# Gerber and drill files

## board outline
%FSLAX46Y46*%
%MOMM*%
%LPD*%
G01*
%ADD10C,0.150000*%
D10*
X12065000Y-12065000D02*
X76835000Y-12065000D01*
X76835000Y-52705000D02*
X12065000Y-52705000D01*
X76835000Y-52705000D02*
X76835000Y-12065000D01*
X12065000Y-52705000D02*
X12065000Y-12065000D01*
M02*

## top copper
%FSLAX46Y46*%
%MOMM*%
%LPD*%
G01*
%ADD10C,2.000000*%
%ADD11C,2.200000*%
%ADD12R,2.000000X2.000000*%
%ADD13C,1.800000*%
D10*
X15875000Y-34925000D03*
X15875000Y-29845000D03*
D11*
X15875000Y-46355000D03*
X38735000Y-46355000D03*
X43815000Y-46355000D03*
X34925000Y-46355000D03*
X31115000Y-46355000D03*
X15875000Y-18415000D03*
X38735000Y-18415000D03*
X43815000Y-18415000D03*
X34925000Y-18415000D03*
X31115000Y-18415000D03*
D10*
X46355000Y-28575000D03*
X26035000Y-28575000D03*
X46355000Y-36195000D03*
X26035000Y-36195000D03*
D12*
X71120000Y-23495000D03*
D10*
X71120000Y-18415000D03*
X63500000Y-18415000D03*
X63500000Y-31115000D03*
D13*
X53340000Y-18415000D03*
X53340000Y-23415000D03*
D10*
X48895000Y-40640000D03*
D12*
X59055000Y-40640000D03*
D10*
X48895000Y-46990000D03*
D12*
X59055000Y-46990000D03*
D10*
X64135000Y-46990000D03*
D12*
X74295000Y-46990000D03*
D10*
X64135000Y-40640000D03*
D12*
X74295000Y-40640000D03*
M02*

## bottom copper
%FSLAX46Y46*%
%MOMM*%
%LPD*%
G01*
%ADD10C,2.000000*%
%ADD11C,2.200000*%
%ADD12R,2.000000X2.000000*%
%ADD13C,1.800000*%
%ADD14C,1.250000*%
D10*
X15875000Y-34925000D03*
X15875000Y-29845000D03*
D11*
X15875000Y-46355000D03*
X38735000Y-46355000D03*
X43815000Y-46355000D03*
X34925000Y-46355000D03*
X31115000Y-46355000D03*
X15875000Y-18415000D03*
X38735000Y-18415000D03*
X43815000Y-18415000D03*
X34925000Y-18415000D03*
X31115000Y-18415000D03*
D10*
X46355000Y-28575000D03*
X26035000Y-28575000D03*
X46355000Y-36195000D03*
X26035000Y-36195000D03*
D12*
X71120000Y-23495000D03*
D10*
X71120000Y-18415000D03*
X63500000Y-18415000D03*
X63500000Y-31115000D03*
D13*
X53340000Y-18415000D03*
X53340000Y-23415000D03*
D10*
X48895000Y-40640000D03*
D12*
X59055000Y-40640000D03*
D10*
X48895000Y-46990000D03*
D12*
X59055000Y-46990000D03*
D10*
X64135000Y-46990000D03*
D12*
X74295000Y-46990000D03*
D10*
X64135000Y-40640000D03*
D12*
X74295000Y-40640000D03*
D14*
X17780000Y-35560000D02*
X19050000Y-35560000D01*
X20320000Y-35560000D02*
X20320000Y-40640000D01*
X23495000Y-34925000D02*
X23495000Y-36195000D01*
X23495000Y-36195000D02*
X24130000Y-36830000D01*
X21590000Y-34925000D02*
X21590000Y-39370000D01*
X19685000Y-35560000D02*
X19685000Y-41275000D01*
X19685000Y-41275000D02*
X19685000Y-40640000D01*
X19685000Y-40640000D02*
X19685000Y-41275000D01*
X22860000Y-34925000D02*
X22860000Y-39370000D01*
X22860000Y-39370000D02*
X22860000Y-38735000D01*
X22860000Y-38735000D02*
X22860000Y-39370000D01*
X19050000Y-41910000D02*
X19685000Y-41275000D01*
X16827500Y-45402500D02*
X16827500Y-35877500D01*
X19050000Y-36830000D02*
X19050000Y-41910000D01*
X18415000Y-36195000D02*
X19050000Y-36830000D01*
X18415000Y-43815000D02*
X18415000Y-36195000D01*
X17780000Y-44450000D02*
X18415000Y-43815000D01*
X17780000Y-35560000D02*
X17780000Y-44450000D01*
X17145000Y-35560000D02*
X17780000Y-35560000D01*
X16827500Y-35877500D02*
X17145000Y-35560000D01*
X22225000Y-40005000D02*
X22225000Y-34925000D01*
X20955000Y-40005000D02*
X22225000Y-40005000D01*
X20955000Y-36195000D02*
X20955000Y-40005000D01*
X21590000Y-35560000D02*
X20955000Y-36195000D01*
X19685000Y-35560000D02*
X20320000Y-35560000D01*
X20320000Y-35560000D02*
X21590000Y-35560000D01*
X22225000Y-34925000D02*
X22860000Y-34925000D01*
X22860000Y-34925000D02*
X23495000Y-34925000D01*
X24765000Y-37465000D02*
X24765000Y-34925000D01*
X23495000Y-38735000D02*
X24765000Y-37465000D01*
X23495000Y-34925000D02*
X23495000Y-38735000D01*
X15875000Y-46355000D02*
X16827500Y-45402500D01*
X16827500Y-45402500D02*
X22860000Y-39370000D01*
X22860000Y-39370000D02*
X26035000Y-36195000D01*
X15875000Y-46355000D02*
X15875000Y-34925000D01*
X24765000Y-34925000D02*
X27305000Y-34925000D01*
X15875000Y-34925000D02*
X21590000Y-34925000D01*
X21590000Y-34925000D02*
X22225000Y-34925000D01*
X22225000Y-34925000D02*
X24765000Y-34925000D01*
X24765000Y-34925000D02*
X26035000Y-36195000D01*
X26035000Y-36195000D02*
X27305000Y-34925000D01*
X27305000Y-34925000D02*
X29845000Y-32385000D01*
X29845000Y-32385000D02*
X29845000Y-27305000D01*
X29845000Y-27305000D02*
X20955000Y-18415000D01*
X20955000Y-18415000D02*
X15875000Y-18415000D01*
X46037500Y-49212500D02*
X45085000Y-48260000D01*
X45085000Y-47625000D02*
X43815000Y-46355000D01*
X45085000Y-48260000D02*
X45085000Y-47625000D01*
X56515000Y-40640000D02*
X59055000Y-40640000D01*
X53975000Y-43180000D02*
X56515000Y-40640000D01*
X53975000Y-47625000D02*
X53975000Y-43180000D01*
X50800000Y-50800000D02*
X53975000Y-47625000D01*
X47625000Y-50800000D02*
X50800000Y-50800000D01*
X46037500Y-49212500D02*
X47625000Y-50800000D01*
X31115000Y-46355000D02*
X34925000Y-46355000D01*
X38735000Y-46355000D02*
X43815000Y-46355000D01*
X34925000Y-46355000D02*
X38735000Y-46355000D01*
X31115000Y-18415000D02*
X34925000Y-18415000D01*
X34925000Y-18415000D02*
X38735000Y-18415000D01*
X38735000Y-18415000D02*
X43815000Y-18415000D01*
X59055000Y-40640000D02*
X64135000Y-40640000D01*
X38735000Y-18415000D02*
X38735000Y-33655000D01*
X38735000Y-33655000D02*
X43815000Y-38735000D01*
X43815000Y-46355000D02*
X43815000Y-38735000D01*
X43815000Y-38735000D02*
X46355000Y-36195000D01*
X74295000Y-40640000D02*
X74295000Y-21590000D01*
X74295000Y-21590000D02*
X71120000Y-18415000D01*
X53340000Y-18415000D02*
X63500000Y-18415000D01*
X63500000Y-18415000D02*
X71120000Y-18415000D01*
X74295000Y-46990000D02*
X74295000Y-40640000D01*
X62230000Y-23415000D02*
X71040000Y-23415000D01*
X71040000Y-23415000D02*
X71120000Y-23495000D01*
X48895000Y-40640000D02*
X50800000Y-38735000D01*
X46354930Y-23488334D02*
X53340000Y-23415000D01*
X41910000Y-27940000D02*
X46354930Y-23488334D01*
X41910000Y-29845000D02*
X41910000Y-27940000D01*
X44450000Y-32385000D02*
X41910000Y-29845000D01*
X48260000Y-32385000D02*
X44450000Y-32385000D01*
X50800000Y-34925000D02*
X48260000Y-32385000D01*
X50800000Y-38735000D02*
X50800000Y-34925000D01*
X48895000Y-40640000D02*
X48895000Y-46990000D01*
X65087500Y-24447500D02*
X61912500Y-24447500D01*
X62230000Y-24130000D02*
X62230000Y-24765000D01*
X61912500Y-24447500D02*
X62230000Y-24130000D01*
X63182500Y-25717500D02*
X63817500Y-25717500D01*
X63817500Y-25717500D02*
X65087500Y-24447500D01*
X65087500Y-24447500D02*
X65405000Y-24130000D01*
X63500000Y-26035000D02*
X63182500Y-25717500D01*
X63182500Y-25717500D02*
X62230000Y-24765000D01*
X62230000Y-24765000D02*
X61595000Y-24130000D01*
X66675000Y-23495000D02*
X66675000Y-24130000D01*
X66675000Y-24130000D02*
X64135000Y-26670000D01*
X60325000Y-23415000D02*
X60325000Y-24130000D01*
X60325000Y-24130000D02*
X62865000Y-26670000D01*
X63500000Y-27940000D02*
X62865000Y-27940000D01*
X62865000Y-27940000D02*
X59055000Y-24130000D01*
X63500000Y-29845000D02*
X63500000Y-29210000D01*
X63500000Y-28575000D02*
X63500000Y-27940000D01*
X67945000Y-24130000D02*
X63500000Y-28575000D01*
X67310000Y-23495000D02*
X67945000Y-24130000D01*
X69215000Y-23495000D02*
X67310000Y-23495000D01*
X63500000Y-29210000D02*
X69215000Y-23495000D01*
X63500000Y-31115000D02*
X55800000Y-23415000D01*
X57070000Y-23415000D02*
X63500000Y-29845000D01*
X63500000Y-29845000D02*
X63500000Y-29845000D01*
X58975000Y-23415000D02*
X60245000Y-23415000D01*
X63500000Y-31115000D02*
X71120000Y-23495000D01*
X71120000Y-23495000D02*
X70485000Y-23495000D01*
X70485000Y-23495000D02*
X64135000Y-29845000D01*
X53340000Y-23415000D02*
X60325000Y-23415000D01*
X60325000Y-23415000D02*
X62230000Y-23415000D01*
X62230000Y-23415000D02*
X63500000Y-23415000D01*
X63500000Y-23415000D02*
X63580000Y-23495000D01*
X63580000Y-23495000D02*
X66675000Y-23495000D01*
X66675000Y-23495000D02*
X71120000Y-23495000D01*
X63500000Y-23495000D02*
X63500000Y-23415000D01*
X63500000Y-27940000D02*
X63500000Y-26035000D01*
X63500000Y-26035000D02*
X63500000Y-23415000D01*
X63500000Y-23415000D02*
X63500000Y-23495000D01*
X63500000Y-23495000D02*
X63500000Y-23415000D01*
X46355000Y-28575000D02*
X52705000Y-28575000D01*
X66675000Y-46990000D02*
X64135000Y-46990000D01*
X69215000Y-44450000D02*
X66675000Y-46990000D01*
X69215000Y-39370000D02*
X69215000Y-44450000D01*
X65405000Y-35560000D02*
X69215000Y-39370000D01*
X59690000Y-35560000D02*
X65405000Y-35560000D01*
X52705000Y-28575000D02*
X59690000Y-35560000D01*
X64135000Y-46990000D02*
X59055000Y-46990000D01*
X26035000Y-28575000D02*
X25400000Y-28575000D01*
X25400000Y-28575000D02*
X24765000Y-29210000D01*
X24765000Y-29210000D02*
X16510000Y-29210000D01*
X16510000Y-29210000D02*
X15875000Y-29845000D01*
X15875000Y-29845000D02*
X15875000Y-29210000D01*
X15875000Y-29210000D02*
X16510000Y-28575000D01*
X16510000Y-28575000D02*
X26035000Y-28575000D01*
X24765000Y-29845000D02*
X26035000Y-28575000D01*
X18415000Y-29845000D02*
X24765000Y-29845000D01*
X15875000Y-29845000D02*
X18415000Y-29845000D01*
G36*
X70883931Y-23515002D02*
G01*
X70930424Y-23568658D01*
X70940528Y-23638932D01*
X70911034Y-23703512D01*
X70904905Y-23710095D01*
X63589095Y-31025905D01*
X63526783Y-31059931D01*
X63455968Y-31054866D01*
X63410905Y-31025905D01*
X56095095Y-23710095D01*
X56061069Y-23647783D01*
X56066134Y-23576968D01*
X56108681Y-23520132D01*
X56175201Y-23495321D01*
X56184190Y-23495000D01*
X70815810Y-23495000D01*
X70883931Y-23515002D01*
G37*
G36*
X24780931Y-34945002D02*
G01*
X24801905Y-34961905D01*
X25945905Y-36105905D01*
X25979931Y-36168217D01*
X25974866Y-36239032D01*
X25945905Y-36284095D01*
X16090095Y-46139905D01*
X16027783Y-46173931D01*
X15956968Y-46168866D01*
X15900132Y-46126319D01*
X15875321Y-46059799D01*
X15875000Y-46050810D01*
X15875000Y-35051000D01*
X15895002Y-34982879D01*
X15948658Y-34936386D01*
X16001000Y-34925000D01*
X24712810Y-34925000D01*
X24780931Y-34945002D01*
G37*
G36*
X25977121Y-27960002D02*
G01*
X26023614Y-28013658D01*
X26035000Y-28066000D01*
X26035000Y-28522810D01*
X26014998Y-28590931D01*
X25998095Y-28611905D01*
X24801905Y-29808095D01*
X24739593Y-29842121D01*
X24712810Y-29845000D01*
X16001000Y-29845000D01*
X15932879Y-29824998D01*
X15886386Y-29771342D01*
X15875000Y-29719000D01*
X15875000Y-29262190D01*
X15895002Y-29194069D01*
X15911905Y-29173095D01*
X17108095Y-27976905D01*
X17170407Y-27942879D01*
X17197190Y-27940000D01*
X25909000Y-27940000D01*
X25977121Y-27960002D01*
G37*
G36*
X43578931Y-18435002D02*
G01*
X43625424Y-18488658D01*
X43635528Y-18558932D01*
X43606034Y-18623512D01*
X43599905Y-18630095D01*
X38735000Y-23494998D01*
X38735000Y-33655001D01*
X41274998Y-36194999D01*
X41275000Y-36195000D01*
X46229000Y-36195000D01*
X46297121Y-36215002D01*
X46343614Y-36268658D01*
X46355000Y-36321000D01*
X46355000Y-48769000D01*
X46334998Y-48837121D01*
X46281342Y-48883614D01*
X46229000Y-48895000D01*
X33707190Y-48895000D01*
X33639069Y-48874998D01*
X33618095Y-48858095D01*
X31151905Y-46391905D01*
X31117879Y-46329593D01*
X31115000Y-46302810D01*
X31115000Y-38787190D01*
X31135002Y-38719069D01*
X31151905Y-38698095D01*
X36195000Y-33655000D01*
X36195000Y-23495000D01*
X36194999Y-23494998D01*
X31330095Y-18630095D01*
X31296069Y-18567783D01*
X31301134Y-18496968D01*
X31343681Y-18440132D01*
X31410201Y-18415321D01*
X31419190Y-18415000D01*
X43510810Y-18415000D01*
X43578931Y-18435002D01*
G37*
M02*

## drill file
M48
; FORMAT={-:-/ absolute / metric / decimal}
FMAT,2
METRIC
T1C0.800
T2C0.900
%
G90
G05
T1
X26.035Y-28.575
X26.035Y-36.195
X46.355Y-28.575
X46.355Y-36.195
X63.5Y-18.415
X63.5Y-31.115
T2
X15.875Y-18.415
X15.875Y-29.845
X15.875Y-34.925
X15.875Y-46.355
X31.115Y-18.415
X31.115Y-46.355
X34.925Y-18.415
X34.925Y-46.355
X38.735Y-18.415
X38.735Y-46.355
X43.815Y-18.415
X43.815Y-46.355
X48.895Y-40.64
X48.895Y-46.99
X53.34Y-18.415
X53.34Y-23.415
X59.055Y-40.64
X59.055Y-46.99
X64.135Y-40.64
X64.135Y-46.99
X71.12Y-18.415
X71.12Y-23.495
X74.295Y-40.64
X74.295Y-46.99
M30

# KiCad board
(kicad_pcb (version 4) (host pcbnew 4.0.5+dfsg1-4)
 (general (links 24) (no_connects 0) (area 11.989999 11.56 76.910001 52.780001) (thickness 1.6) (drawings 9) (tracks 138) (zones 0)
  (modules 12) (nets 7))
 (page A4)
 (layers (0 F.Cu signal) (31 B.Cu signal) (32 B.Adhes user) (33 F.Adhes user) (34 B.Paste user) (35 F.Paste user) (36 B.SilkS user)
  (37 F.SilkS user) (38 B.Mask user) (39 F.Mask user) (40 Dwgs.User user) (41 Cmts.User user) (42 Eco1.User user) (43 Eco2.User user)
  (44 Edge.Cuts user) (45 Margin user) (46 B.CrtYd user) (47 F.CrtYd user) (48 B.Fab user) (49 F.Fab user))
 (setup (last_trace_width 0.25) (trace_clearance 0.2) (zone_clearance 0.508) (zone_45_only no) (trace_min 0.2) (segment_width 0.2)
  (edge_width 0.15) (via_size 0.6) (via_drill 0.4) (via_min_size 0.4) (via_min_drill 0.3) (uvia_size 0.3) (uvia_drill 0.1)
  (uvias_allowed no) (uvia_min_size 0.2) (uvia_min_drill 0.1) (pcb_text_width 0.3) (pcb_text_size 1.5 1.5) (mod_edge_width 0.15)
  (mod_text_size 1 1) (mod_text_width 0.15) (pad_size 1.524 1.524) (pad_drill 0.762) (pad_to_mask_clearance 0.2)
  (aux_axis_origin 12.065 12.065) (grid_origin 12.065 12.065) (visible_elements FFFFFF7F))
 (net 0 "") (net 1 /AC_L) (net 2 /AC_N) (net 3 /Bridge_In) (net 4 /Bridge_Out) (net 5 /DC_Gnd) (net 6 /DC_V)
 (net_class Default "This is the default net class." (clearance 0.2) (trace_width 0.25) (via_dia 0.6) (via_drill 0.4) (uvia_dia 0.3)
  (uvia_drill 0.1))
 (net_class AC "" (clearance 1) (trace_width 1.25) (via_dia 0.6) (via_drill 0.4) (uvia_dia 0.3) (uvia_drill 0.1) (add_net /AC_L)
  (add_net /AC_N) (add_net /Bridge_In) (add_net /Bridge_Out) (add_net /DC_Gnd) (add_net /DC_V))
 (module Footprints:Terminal (layer F.Cu) (at 15.875 32.385)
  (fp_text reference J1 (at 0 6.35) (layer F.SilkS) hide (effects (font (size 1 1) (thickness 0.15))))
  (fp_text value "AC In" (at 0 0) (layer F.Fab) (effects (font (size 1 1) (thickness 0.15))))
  (pad 1 thru_hole circle (at 0 2.54) (size 2 2) (drill 0.9) (layers *.Cu *.Mask) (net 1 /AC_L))
  (pad 2 thru_hole circle (at 0 -2.54) (size 2 2) (drill 0.9) (layers *.Cu *.Mask) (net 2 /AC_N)))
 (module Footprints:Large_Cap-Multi (layer F.Cu) (at 31.115 43.815)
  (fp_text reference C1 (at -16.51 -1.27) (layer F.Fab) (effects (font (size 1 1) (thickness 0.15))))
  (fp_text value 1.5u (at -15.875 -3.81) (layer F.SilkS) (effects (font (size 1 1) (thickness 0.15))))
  (pad 1 thru_hole circle (at -15.24 2.54) (size 2.2 2.2) (drill 0.9) (layers *.Cu *.Mask) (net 1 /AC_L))
  (pad 2 thru_hole circle (at 7.62 2.54) (size 2.2 2.2) (drill 0.9) (layers *.Cu *.Mask) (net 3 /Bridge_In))
  (pad 2 thru_hole circle (at 12.7 2.54) (size 2.2 2.2) (drill 0.9) (layers *.Cu *.Mask) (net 3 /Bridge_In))
  (pad 2 thru_hole circle (at 3.81 2.54) (size 2.2 2.2) (drill 0.9) (layers *.Cu *.Mask) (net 3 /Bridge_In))
  (pad 2 thru_hole circle (at 0 2.54) (size 2.2 2.2) (drill 0.9) (layers *.Cu *.Mask) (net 3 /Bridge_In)))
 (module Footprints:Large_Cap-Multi (layer F.Cu) (at 31.115 15.875)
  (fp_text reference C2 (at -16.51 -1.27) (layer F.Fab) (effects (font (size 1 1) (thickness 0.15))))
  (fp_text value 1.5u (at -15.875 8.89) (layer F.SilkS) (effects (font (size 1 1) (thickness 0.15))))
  (pad 1 thru_hole circle (at -15.24 2.54) (size 2.2 2.2) (drill 0.9) (layers *.Cu *.Mask) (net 1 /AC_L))
  (pad 2 thru_hole circle (at 7.62 2.54) (size 2.2 2.2) (drill 0.9) (layers *.Cu *.Mask) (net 3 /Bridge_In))
  (pad 2 thru_hole circle (at 12.7 2.54) (size 2.2 2.2) (drill 0.9) (layers *.Cu *.Mask) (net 3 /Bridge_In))
  (pad 2 thru_hole circle (at 3.81 2.54) (size 2.2 2.2) (drill 0.9) (layers *.Cu *.Mask) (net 3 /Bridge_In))
  (pad 2 thru_hole circle (at 0 2.54) (size 2.2 2.2) (drill 0.9) (layers *.Cu *.Mask) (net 3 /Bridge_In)))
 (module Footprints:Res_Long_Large (layer F.Cu) (at 36.195 28.575 180)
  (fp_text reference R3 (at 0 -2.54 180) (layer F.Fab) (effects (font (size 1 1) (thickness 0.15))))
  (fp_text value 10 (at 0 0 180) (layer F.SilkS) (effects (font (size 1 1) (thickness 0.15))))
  (pad 1 thru_hole circle (at -10.16 0 180) (size 2 2) (drill 0.8) (layers *.Cu *.Mask) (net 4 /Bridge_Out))
  (pad 2 thru_hole circle (at 10.16 0 180) (size 2 2) (drill 0.8) (layers *.Cu *.Mask) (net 2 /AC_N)))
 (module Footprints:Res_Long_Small (layer F.Cu) (at 36.195 36.195 180)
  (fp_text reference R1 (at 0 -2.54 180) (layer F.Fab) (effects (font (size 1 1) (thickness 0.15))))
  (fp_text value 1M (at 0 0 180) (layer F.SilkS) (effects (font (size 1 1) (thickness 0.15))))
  (pad 1 thru_hole circle (at -10.16 0 180) (size 2 2) (drill 0.8) (layers *.Cu *.Mask) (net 3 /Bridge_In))
  (pad 2 thru_hole circle (at 10.16 0 180) (size 2 2) (drill 0.8) (layers *.Cu *.Mask) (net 1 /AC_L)))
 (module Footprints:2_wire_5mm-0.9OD (layer F.Cu) (at 71.12 20.955 90)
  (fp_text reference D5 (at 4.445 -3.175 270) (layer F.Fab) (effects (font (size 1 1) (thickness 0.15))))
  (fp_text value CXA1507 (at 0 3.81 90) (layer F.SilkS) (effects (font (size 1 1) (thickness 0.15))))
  (pad 1 thru_hole rect (at -2.54 0 90) (size 2 2) (drill 0.9) (layers *.Cu *.Mask) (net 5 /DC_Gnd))
  (pad 2 thru_hole circle (at 2.54 0 90) (size 2 2) (drill 0.9) (layers *.Cu *.Mask) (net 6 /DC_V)))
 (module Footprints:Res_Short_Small (layer F.Cu) (at 63.5 24.765 270)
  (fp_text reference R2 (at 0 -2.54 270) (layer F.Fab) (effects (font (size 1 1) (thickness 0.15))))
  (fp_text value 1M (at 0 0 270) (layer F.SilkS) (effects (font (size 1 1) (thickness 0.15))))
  (pad 1 thru_hole circle (at -6.35 0 270) (size 2 2) (drill 0.8) (layers *.Cu *.Mask) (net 6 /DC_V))
  (pad 2 thru_hole circle (at 6.35 0 270) (size 2 2) (drill 0.8) (layers *.Cu *.Mask) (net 5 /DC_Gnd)))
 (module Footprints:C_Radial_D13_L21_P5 (layer F.Cu) (at 53.34 18.415 270)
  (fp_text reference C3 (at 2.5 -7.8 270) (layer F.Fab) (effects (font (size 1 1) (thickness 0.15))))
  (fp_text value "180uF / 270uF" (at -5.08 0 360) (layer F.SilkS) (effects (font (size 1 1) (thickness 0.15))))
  (pad 1 thru_hole circle (at 0 0 270) (size 1.8 1.8) (drill 0.9) (layers *.Cu *.Mask) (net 6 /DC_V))
  (pad 2 thru_hole circle (at 5 0 270) (size 1.8 1.8) (drill 0.9) (layers *.Cu *.Mask) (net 5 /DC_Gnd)))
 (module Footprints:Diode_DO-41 (layer F.Cu) (at 59.055 40.64 180)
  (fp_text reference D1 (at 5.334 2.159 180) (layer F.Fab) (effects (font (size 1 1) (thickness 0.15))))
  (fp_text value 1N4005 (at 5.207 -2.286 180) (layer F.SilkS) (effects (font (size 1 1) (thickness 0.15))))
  (pad 2 thru_hole circle (at 10.16 0) (size 2 2) (drill 0.9) (layers *.Cu *.Mask) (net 5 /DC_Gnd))
  (pad 1 thru_hole rect (at 0 0) (size 2 2) (drill 0.9) (layers *.Cu *.Mask) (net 3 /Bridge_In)))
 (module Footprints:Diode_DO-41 (layer F.Cu) (at 59.055 46.99 180)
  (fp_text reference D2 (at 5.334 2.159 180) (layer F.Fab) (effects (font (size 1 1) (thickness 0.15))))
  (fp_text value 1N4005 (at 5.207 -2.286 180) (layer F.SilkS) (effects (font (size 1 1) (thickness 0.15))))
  (pad 2 thru_hole circle (at 10.16 0) (size 2 2) (drill 0.9) (layers *.Cu *.Mask) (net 5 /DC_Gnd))
  (pad 1 thru_hole rect (at 0 0) (size 2 2) (drill 0.9) (layers *.Cu *.Mask) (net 4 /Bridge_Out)))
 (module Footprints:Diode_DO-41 (layer F.Cu) (at 74.295 46.99 180)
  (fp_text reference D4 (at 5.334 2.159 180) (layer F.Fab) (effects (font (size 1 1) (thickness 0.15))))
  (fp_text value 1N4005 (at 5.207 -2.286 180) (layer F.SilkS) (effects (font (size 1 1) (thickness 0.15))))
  (pad 2 thru_hole circle (at 10.16 0) (size 2 2) (drill 0.9) (layers *.Cu *.Mask) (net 4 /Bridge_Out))
  (pad 1 thru_hole rect (at 0 0) (size 2 2) (drill 0.9) (layers *.Cu *.Mask) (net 6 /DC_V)))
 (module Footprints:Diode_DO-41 (layer F.Cu) (at 74.295 40.64 180)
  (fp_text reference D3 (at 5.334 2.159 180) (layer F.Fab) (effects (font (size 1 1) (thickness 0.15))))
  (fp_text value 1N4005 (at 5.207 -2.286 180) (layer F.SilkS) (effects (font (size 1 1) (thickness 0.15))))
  (pad 2 thru_hole circle (at 10.16 0) (size 2 2) (drill 0.9) (layers *.Cu *.Mask) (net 3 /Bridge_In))
  (pad 1 thru_hole rect (at 0 0) (size 2 2) (drill 0.9) (layers *.Cu *.Mask) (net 6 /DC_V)))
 (gr_line (start 12.065 12.065) (end 76.835 12.065) (angle 90) (layer Edge.Cuts) (width 0.15))
 (gr_line (start 76.835 52.705) (end 12.065 52.705) (angle 90) (layer Edge.Cuts) (width 0.15))
 (gr_line (start 76.835 52.705) (end 76.835 12.065) (angle 90) (layer Edge.Cuts) (width 0.15))
 (gr_line (start 12.065 52.705) (end 12.065 12.065) (angle 90) (layer Edge.Cuts) (width 0.15))
 (segment (start 17.78 35.56) (end 19.05 35.56) (width 1.25) (layer B.Cu) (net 1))
 (segment (start 20.32 35.56) (end 20.32 40.64) (width 1.25) (layer B.Cu) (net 1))
 (segment (start 23.495 34.925) (end 23.495 36.195) (width 1.25) (layer B.Cu) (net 1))
 (segment (start 23.495 36.195) (end 24.13 36.83) (width 1.25) (layer B.Cu) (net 1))
 (segment (start 21.59 34.925) (end 21.59 39.37) (width 1.25) (layer B.Cu) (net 1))
 (segment (start 19.685 35.56) (end 19.685 41.275) (width 1.25) (layer B.Cu) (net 1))
 (segment (start 19.685 41.275) (end 19.685 40.64) (width 1.25) (layer B.Cu) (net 1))
 (segment (start 19.685 40.64) (end 19.685 41.275) (width 1.25) (layer B.Cu) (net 1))
 (segment (start 22.86 34.925) (end 22.86 39.37) (width 1.25) (layer B.Cu) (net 1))
 (segment (start 22.86 39.37) (end 22.86 38.735) (width 1.25) (layer B.Cu) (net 1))
 (segment (start 22.86 38.735) (end 22.86 39.37) (width 1.25) (layer B.Cu) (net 1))
 (segment (start 19.05 41.91) (end 19.685 41.275) (width 1.25) (layer B.Cu) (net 1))
 (segment (start 16.8275 45.4025) (end 16.8275 35.8775) (width 1.25) (layer B.Cu) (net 1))
 (segment (start 19.05 36.83) (end 19.05 41.91) (width 1.25) (layer B.Cu) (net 1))
 (segment (start 18.415 36.195) (end 19.05 36.83) (width 1.25) (layer B.Cu) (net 1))
 (segment (start 18.415 43.815) (end 18.415 36.195) (width 1.25) (layer B.Cu) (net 1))
 (segment (start 17.78 44.45) (end 18.415 43.815) (width 1.25) (layer B.Cu) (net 1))
 (segment (start 17.78 35.56) (end 17.78 44.45) (width 1.25) (layer B.Cu) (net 1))
 (segment (start 17.145 35.56) (end 17.78 35.56) (width 1.25) (layer B.Cu) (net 1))
 (segment (start 16.8275 35.8775) (end 17.145 35.56) (width 1.25) (layer B.Cu) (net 1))
 (segment (start 22.225 40.005) (end 22.225 34.925) (width 1.25) (layer B.Cu) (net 1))
 (segment (start 20.955 40.005) (end 22.225 40.005) (width 1.25) (layer B.Cu) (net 1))
 (segment (start 20.955 36.195) (end 20.955 40.005) (width 1.25) (layer B.Cu) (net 1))
 (segment (start 21.59 35.56) (end 20.955 36.195) (width 1.25) (layer B.Cu) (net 1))
 (segment (start 19.685 35.56) (end 20.32 35.56) (width 1.25) (layer B.Cu) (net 1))
 (segment (start 20.32 35.56) (end 21.59 35.56) (width 1.25) (layer B.Cu) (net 1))
 (segment (start 22.225 34.925) (end 22.86 34.925) (width 1.25) (layer B.Cu) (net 1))
 (segment (start 22.86 34.925) (end 23.495 34.925) (width 1.25) (layer B.Cu) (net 1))
 (segment (start 24.765 37.465) (end 24.765 34.925) (width 1.25) (layer B.Cu) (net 1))
 (segment (start 23.495 38.735) (end 24.765 37.465) (width 1.25) (layer B.Cu) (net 1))
 (segment (start 23.495 34.925) (end 23.495 38.735) (width 1.25) (layer B.Cu) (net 1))
 (segment (start 15.875 46.355) (end 16.8275 45.4025) (width 1.25) (layer B.Cu) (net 1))
 (segment (start 16.8275 45.4025) (end 22.86 39.37) (width 1.25) (layer B.Cu) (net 1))
 (segment (start 22.86 39.37) (end 26.035 36.195) (width 1.25) (layer B.Cu) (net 1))
 (segment (start 15.875 46.355) (end 15.875 34.925) (width 1.25) (layer B.Cu) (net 1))
 (segment (start 24.765 34.925) (end 27.305 34.925) (width 1.25) (layer B.Cu) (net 1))
 (segment (start 15.875 34.925) (end 21.59 34.925) (width 1.25) (layer B.Cu) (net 1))
 (segment (start 21.59 34.925) (end 22.225 34.925) (width 1.25) (layer B.Cu) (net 1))
 (segment (start 22.225 34.925) (end 24.765 34.925) (width 1.25) (layer B.Cu) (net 1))
 (segment (start 24.765 34.925) (end 26.035 36.195) (width 1.25) (layer B.Cu) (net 1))
 (segment (start 26.035 36.195) (end 27.305 34.925) (width 1.25) (layer B.Cu) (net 1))
 (segment (start 27.305 34.925) (end 29.845 32.385) (width 1.25) (layer B.Cu) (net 1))
 (segment (start 29.845 32.385) (end 29.845 27.305) (width 1.25) (layer B.Cu) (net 1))
 (segment (start 29.845 27.305) (end 20.955 18.415) (width 1.25) (layer B.Cu) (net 1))
 (segment (start 20.955 18.415) (end 15.875 18.415) (width 1.25) (layer B.Cu) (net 1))
 (segment (start 46.0375 49.2125) (end 45.085 48.26) (width 1.25) (layer B.Cu) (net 3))
 (segment (start 45.085 47.625) (end 43.815 46.355) (width 1.25) (layer B.Cu) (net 3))
 (segment (start 45.085 48.26) (end 45.085 47.625) (width 1.25) (layer B.Cu) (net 3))
 (segment (start 56.515 40.64) (end 59.055 40.64) (width 1.25) (layer B.Cu) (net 3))
 (segment (start 53.975 43.18) (end 56.515 40.64) (width 1.25) (layer B.Cu) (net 3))
 (segment (start 53.975 47.625) (end 53.975 43.18) (width 1.25) (layer B.Cu) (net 3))
 (segment (start 50.8 50.8) (end 53.975 47.625) (width 1.25) (layer B.Cu) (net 3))
 (segment (start 47.625 50.8) (end 50.8 50.8) (width 1.25) (layer B.Cu) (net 3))
 (segment (start 46.0375 49.2125) (end 47.625 50.8) (width 1.25) (layer B.Cu) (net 3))
 (segment (start 31.115 46.355) (end 34.925 46.355) (width 1.25) (layer B.Cu) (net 3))
 (segment (start 38.735 46.355) (end 43.815 46.355) (width 1.25) (layer B.Cu) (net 3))
 (segment (start 34.925 46.355) (end 38.735 46.355) (width 1.25) (layer B.Cu) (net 3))
 (segment (start 31.115 18.415) (end 34.925 18.415) (width 1.25) (layer B.Cu) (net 3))
 (segment (start 34.925 18.415) (end 38.735 18.415) (width 1.25) (layer B.Cu) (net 3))
 (segment (start 38.735 18.415) (end 43.815 18.415) (width 1.25) (layer B.Cu) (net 3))
 (segment (start 59.055 40.64) (end 64.135 40.64) (width 1.25) (layer B.Cu) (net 3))
 (segment (start 38.735 18.415) (end 38.735 33.655) (width 1.25) (layer B.Cu) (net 3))
 (segment (start 38.735 33.655) (end 43.815 38.735) (width 1.25) (layer B.Cu) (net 3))
 (segment (start 43.815 46.355) (end 43.815 38.735) (width 1.25) (layer B.Cu) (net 3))
 (segment (start 43.815 38.735) (end 46.355 36.195) (width 1.25) (layer B.Cu) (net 3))
 (segment (start 74.295 40.64) (end 74.295 21.59) (width 1.25) (layer B.Cu) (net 6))
 (segment (start 74.295 21.59) (end 71.12 18.415) (width 1.25) (layer B.Cu) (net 6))
 (segment (start 53.34 18.415) (end 63.5 18.415) (width 1.25) (layer B.Cu) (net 6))
 (segment (start 63.5 18.415) (end 71.12 18.415) (width 1.25) (layer B.Cu) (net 6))
 (segment (start 74.295 46.99) (end 74.295 40.64) (width 1.25) (layer B.Cu) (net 6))
 (segment (start 62.23 23.415) (end 71.04 23.415) (width 1.25) (layer B.Cu) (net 5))
 (segment (start 71.04 23.415) (end 71.12 23.495) (width 1.25) (layer B.Cu) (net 5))
 (segment (start 48.895 40.64) (end 50.8 38.735) (width 1.25) (layer B.Cu) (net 5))
 (segment (start 46.35493 23.488334) (end 53.34 23.415) (width 1.25) (layer B.Cu) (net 5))
 (segment (start 41.91 27.94) (end 46.35493 23.488334) (width 1.25) (layer B.Cu) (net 5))
 (segment (start 41.91 29.845) (end 41.91 27.94) (width 1.25) (layer B.Cu) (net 5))
 (segment (start 44.45 32.385) (end 41.91 29.845) (width 1.25) (layer B.Cu) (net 5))
 (segment (start 48.26 32.385) (end 44.45 32.385) (width 1.25) (layer B.Cu) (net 5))
 (segment (start 50.8 34.925) (end 48.26 32.385) (width 1.25) (layer B.Cu) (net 5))
 (segment (start 50.8 38.735) (end 50.8 34.925) (width 1.25) (layer B.Cu) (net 5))
 (segment (start 48.895 40.64) (end 48.895 46.99) (width 1.25) (layer B.Cu) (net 5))
 (segment (start 65.0875 24.4475) (end 61.9125 24.4475) (width 1.25) (layer B.Cu) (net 5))
 (segment (start 62.23 24.13) (end 62.23 24.765) (width 1.25) (layer B.Cu) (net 5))
 (segment (start 61.9125 24.4475) (end 62.23 24.13) (width 1.25) (layer B.Cu) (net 5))
 (segment (start 63.1825 25.7175) (end 63.8175 25.7175) (width 1.25) (layer B.Cu) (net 5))
 (segment (start 63.8175 25.7175) (end 65.0875 24.4475) (width 1.25) (layer B.Cu) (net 5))
 (segment (start 65.0875 24.4475) (end 65.405 24.13) (width 1.25) (layer B.Cu) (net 5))
 (segment (start 63.5 26.035) (end 63.1825 25.7175) (width 1.25) (layer B.Cu) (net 5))
 (segment (start 63.1825 25.7175) (end 62.23 24.765) (width 1.25) (layer B.Cu) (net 5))
 (segment (start 62.23 24.765) (end 61.595 24.13) (width 1.25) (layer B.Cu) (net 5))
 (segment (start 66.675 23.495) (end 66.675 24.13) (width 1.25) (layer B.Cu) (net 5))
 (segment (start 66.675 24.13) (end 64.135 26.67) (width 1.25) (layer B.Cu) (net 5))
 (segment (start 60.325 23.415) (end 60.325 24.13) (width 1.25) (layer B.Cu) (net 5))
 (segment (start 60.325 24.13) (end 62.865 26.67) (width 1.25) (layer B.Cu) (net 5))
 (segment (start 63.5 27.94) (end 62.865 27.94) (width 1.25) (layer B.Cu) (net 5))
 (segment (start 62.865 27.94) (end 59.055 24.13) (width 1.25) (layer B.Cu) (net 5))
 (segment (start 63.5 29.845) (end 63.5 29.21) (width 1.25) (layer B.Cu) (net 5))
 (segment (start 63.5 28.575) (end 63.5 27.94) (width 1.25) (layer B.Cu) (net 5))
 (segment (start 67.945 24.13) (end 63.5 28.575) (width 1.25) (layer B.Cu) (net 5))
 (segment (start 67.31 23.495) (end 67.945 24.13) (width 1.25) (layer B.Cu) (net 5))
 (segment (start 69.215 23.495) (end 67.31 23.495) (width 1.25) (layer B.Cu) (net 5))
 (segment (start 63.5 29.21) (end 69.215 23.495) (width 1.25) (layer B.Cu) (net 5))
 (segment (start 63.5 31.115) (end 55.8 23.415) (width 1.25) (layer B.Cu) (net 5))
 (segment (start 57.07 23.415) (end 63.5 29.845) (width 1.25) (layer B.Cu) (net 5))
 (segment (start 63.5 29.845) (end 63.5 29.845) (width 1.25) (layer B.Cu) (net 5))
 (segment (start 58.975 23.415) (end 60.245 23.415) (width 1.25) (layer B.Cu) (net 5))
 (segment (start 63.5 31.115) (end 71.12 23.495) (width 1.25) (layer B.Cu) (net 5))
 (segment (start 71.12 23.495) (end 70.485 23.495) (width 1.25) (layer B.Cu) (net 5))
 (segment (start 70.485 23.495) (end 64.135 29.845) (width 1.25) (layer B.Cu) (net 5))
 (segment (start 53.34 23.415) (end 60.325 23.415) (width 1.25) (layer B.Cu) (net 5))
 (segment (start 60.325 23.415) (end 62.23 23.415) (width 1.25) (layer B.Cu) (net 5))
 (segment (start 62.23 23.415) (end 63.5 23.415) (width 1.25) (layer B.Cu) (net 5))
 (segment (start 63.5 23.415) (end 63.58 23.495) (width 1.25) (layer B.Cu) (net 5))
 (segment (start 63.58 23.495) (end 66.675 23.495) (width 1.25) (layer B.Cu) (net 5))
 (segment (start 66.675 23.495) (end 71.12 23.495) (width 1.25) (layer B.Cu) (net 5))
 (segment (start 63.5 23.495) (end 63.5 23.415) (width 1.25) (layer B.Cu) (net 5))
 (segment (start 63.5 27.94) (end 63.5 26.035) (width 1.25) (layer B.Cu) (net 5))
 (segment (start 63.5 26.035) (end 63.5 23.415) (width 1.25) (layer B.Cu) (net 5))
 (segment (start 63.5 23.415) (end 63.5 23.495) (width 1.25) (layer B.Cu) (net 5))
 (segment (start 63.5 23.495) (end 63.5 23.415) (width 1.25) (layer B.Cu) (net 5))
 (segment (start 46.355 28.575) (end 52.705 28.575) (width 1.25) (layer B.Cu) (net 4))
 (segment (start 66.675 46.99) (end 64.135 46.99) (width 1.25) (layer B.Cu) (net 4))
 (segment (start 69.215 44.45) (end 66.675 46.99) (width 1.25) (layer B.Cu) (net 4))
 (segment (start 69.215 39.37) (end 69.215 44.45) (width 1.25) (layer B.Cu) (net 4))
 (segment (start 65.405 35.56) (end 69.215 39.37) (width 1.25) (layer B.Cu) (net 4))
 (segment (start 59.69 35.56) (end 65.405 35.56) (width 1.25) (layer B.Cu) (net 4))
 (segment (start 52.705 28.575) (end 59.69 35.56) (width 1.25) (layer B.Cu) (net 4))
 (segment (start 64.135 46.99) (end 59.055 46.99) (width 1.25) (layer B.Cu) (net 4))
 (segment (start 26.035 28.575) (end 25.4 28.575) (width 1.25) (layer B.Cu) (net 2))
 (segment (start 25.4 28.575) (end 24.765 29.21) (width 1.25) (layer B.Cu) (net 2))
 (segment (start 24.765 29.21) (end 16.51 29.21) (width 1.25) (layer B.Cu) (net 2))
 (segment (start 16.51 29.21) (end 15.875 29.845) (width 1.25) (layer B.Cu) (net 2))
 (segment (start 15.875 29.845) (end 15.875 29.21) (width 1.25) (layer B.Cu) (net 2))
 (segment (start 15.875 29.21) (end 16.51 28.575) (width 1.25) (layer B.Cu) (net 2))
 (segment (start 16.51 28.575) (end 26.035 28.575) (width 1.25) (layer B.Cu) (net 2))
 (segment (start 24.765 29.845) (end 26.035 28.575) (width 1.25) (layer B.Cu) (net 2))
 (segment (start 18.415 29.845) (end 24.765 29.845) (width 1.25) (layer B.Cu) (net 2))
 (segment (start 15.875 29.845) (end 18.415 29.845) (width 1.25) (layer B.Cu) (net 2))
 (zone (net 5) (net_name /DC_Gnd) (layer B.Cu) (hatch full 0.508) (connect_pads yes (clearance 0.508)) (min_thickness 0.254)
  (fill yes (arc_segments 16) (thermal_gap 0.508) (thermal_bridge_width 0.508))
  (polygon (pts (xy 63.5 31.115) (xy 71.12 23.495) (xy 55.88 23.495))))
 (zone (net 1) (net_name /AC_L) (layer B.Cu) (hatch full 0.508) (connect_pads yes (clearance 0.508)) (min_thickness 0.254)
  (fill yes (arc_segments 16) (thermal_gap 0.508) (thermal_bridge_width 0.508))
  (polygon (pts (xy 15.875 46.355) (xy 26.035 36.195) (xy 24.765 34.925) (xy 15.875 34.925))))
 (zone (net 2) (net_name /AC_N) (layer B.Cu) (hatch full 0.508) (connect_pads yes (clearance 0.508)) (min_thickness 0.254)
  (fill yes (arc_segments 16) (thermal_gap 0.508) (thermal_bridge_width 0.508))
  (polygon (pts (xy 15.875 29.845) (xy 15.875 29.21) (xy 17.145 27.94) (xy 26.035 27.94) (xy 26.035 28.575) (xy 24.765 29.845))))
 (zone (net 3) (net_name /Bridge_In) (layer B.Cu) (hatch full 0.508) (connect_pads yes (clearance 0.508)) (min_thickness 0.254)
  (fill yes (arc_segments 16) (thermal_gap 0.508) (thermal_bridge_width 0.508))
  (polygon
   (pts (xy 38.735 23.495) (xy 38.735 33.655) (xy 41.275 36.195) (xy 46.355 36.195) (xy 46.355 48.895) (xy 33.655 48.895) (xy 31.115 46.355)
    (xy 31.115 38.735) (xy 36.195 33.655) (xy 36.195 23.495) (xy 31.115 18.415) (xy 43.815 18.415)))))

